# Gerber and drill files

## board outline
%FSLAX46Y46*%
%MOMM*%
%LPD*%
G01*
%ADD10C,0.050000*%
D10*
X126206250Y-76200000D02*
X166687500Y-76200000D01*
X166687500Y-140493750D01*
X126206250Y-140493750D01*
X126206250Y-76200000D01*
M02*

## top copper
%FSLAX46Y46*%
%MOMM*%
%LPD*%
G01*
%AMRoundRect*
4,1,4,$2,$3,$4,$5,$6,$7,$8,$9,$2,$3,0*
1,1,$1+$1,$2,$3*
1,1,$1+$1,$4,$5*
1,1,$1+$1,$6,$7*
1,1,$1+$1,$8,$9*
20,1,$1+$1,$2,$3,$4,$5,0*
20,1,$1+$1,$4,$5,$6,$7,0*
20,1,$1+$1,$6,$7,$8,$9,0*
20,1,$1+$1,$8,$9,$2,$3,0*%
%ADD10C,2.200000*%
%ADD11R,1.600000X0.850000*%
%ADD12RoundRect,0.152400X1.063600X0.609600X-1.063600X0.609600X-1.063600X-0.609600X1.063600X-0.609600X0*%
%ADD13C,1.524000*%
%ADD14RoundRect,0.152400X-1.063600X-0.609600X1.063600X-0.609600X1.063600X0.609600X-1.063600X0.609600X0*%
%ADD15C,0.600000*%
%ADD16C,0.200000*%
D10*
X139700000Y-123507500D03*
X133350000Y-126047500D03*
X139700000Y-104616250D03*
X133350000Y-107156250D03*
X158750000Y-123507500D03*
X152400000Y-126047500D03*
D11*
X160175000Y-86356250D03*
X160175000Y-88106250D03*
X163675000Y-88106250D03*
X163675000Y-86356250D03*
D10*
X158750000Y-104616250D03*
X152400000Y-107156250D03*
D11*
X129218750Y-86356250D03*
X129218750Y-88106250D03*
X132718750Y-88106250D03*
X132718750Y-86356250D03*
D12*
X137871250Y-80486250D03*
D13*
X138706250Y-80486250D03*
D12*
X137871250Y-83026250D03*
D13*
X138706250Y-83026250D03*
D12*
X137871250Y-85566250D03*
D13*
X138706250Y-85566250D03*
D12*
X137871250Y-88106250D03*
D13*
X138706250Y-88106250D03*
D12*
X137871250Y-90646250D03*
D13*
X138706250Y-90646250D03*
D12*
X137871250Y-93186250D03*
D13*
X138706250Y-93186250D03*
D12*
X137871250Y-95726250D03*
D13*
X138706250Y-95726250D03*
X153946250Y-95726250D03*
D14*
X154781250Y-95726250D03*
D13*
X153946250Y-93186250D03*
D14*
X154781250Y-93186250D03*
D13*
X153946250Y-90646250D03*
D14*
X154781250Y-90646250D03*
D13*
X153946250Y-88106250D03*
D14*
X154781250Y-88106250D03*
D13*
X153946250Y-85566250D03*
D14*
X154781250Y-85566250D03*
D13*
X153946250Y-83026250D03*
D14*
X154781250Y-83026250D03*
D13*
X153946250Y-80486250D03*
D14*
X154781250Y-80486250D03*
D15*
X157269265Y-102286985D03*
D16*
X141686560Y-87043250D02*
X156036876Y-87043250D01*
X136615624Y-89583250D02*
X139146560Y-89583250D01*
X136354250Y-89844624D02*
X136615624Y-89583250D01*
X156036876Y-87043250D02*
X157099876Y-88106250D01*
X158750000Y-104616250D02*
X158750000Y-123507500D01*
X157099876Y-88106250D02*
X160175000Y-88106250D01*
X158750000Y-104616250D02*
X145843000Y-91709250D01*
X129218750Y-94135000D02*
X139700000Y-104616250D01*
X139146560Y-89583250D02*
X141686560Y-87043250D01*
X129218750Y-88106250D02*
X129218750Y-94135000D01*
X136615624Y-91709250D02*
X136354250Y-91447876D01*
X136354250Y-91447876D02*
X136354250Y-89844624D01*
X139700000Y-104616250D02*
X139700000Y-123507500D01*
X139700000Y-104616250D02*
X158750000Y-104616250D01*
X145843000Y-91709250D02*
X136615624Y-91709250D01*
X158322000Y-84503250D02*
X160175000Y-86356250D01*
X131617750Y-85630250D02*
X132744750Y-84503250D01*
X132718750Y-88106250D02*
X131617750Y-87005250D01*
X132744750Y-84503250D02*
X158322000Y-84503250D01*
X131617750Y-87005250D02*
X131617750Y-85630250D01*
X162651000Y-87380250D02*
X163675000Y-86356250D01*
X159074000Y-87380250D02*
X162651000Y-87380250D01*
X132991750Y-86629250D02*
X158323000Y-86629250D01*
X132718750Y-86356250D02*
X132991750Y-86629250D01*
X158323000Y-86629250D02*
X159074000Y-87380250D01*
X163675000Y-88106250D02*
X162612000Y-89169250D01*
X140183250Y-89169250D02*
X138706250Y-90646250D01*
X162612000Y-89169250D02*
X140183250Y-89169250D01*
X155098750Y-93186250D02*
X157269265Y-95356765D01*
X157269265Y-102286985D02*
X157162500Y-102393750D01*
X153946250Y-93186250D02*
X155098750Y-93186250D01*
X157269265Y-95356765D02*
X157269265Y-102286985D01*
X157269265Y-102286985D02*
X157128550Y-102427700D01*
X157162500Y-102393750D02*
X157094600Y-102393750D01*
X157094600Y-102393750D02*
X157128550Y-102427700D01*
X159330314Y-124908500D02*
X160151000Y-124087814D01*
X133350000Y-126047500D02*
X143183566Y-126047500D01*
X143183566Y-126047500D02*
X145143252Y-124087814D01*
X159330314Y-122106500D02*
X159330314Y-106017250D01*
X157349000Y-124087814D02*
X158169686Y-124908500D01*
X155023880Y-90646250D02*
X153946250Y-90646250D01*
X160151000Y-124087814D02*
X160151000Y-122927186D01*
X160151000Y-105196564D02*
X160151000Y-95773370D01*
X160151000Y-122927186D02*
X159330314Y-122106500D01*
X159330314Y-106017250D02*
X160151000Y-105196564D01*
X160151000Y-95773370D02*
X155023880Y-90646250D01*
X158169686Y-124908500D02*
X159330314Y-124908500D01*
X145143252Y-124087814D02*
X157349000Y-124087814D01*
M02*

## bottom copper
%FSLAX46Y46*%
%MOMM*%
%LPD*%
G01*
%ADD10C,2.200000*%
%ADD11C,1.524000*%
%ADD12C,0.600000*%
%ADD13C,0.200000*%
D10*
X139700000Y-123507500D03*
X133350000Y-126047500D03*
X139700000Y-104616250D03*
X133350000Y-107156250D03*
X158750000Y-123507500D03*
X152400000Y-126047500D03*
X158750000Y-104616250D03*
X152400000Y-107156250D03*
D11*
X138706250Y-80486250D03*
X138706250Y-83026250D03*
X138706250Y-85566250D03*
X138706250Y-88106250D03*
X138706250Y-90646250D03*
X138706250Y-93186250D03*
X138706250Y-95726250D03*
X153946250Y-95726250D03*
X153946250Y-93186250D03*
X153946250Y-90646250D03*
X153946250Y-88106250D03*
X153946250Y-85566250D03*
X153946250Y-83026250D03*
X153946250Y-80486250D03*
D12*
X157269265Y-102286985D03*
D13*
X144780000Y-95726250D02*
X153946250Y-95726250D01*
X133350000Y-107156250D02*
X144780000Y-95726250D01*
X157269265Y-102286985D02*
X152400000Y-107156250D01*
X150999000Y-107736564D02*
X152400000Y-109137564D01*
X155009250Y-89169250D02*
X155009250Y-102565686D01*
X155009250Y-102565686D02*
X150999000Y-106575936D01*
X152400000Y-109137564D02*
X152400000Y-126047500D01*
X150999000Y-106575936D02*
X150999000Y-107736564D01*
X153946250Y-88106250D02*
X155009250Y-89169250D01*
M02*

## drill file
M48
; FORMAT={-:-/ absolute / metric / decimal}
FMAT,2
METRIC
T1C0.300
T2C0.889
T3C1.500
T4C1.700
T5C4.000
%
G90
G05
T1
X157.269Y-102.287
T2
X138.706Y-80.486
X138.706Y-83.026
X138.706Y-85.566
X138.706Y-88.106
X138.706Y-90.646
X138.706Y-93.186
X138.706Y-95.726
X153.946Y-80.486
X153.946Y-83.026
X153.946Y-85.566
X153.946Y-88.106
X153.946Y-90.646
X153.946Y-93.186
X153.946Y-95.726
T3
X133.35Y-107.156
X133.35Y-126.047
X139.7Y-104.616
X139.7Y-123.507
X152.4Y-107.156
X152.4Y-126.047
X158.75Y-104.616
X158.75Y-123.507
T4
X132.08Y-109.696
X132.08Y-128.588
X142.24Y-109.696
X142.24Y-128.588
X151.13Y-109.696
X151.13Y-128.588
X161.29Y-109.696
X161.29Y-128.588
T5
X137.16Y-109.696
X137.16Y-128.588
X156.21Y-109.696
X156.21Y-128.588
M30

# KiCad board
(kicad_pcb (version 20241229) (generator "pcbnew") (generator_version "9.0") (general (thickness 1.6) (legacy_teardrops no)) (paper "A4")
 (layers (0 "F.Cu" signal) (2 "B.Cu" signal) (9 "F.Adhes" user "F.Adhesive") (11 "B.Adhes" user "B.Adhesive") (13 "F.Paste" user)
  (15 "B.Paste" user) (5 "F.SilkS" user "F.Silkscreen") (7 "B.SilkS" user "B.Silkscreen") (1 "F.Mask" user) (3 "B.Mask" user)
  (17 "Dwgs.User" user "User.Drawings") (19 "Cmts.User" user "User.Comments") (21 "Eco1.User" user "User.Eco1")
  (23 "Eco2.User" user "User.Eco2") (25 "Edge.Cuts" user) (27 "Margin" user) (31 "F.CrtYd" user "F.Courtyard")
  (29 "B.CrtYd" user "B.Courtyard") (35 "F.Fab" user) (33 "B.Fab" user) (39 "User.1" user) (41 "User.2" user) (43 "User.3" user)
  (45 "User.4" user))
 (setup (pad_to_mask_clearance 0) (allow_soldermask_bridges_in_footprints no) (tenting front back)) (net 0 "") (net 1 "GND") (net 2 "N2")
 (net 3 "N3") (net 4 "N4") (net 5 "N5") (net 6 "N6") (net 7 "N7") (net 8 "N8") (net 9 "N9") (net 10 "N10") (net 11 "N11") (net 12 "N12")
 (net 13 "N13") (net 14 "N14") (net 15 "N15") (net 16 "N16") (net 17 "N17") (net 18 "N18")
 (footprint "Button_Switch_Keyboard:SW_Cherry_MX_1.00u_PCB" (layer "F.Cu") (at 139.7 123.5075)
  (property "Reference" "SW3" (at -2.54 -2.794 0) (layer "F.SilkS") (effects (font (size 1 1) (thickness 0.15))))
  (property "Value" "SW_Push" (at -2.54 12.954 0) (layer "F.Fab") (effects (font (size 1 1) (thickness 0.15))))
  (pad "" np_thru_hole circle (at -7.62 5.08) (size 1.7 1.7) (drill 1.7) (layers "*.Cu" "*.Mask"))
  (pad "" np_thru_hole circle (at -2.54 5.08) (size 4 4) (drill 4) (layers "*.Cu" "*.Mask"))
  (pad "" np_thru_hole circle (at 2.54 5.08) (size 1.7 1.7) (drill 1.7) (layers "*.Cu" "*.Mask"))
  (pad "1" thru_hole circle (at 0 0) (size 2.2 2.2) (drill 1.5) (layers "*.Cu" "*.Mask") (remove_unused_layers no) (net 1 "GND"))
  (pad "2" thru_hole circle (at -6.35 2.54) (size 2.2 2.2) (drill 1.5) (layers "*.Cu" "*.Mask") (remove_unused_layers no) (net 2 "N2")))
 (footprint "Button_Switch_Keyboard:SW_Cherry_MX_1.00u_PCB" (layer "F.Cu") (at 139.7 104.61625)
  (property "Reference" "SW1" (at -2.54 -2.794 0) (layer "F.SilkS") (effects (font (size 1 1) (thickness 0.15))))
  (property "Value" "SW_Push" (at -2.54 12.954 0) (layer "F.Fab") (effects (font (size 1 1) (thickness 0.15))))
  (pad "" np_thru_hole circle (at -7.62 5.08) (size 1.7 1.7) (drill 1.7) (layers "*.Cu" "*.Mask"))
  (pad "" np_thru_hole circle (at -2.54 5.08) (size 4 4) (drill 4) (layers "*.Cu" "*.Mask"))
  (pad "" np_thru_hole circle (at 2.54 5.08) (size 1.7 1.7) (drill 1.7) (layers "*.Cu" "*.Mask"))
  (pad "1" thru_hole circle (at 0 0) (size 2.2 2.2) (drill 1.5) (layers "*.Cu" "*.Mask") (remove_unused_layers no) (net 1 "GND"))
  (pad "2" thru_hole circle (at -6.35 2.54) (size 2.2 2.2) (drill 1.5) (layers "*.Cu" "*.Mask") (remove_unused_layers no) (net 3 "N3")))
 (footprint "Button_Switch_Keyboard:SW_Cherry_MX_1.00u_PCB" (layer "F.Cu") (at 158.75 123.5075)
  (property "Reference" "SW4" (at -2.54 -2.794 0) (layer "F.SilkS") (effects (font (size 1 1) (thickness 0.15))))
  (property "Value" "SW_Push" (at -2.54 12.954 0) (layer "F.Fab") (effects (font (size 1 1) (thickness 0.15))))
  (pad "" np_thru_hole circle (at -7.62 5.08) (size 1.7 1.7) (drill 1.7) (layers "*.Cu" "*.Mask"))
  (pad "" np_thru_hole circle (at -2.54 5.08) (size 4 4) (drill 4) (layers "*.Cu" "*.Mask"))
  (pad "" np_thru_hole circle (at 2.54 5.08) (size 1.7 1.7) (drill 1.7) (layers "*.Cu" "*.Mask"))
  (pad "1" thru_hole circle (at 0 0) (size 2.2 2.2) (drill 1.5) (layers "*.Cu" "*.Mask") (remove_unused_layers no) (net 1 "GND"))
  (pad "2" thru_hole circle (at -6.35 2.54) (size 2.2 2.2) (drill 1.5) (layers "*.Cu" "*.Mask") (remove_unused_layers no) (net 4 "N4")))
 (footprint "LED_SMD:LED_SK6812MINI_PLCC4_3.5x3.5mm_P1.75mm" (layer "F.Cu") (at 161.925 87.23125)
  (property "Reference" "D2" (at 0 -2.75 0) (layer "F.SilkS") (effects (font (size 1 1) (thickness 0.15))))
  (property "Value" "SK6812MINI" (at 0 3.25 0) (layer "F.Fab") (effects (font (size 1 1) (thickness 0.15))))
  (pad "1" smd rect (at -1.75 -0.875) (size 1.6 0.85) (layers "F.Cu" "F.Mask" "F.Paste") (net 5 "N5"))
  (pad "2" smd rect (at -1.75 0.875) (size 1.6 0.85) (layers "F.Cu" "F.Mask" "F.Paste") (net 1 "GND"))
  (pad "3" smd rect (at 1.75 0.875) (size 1.6 0.85) (layers "F.Cu" "F.Mask" "F.Paste") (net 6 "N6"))
  (pad "4" smd rect (at 1.75 -0.875) (size 1.6 0.85) (layers "F.Cu" "F.Mask" "F.Paste") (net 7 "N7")))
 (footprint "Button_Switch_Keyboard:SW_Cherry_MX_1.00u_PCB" (layer "F.Cu") (at 158.75 104.61625)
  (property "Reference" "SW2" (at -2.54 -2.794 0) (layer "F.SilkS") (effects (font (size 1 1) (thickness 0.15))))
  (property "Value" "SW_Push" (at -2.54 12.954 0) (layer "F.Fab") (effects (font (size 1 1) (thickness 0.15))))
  (pad "" np_thru_hole circle (at -7.62 5.08) (size 1.7 1.7) (drill 1.7) (layers "*.Cu" "*.Mask"))
  (pad "" np_thru_hole circle (at -2.54 5.08) (size 4 4) (drill 4) (layers "*.Cu" "*.Mask"))
  (pad "" np_thru_hole circle (at 2.54 5.08) (size 1.7 1.7) (drill 1.7) (layers "*.Cu" "*.Mask"))
  (pad "1" thru_hole circle (at 0 0) (size 2.2 2.2) (drill 1.5) (layers "*.Cu" "*.Mask") (remove_unused_layers no) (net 1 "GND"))
  (pad "2" thru_hole circle (at -6.35 2.54) (size 2.2 2.2) (drill 1.5) (layers "*.Cu" "*.Mask") (remove_unused_layers no) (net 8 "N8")))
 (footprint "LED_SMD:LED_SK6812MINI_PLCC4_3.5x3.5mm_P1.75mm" (layer "F.Cu") (at 130.96875 87.23125)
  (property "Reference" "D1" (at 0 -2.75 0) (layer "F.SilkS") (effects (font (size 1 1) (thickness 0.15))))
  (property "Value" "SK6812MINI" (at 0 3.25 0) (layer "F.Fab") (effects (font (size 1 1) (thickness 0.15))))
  (pad "1" smd rect (at -1.75 -0.875) (size 1.6 0.85) (layers "F.Cu" "F.Mask" "F.Paste") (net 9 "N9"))
  (pad "2" smd rect (at -1.75 0.875) (size 1.6 0.85) (layers "F.Cu" "F.Mask" "F.Paste") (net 1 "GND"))
  (pad "3" smd rect (at 1.75 0.875) (size 1.6 0.85) (layers "F.Cu" "F.Mask" "F.Paste") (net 5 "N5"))
  (pad "4" smd rect (at 1.75 -0.875) (size 1.6 0.85) (layers "F.Cu" "F.Mask" "F.Paste") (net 7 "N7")))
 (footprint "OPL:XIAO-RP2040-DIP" (layer "F.Cu") (at 146.32625 88.10625)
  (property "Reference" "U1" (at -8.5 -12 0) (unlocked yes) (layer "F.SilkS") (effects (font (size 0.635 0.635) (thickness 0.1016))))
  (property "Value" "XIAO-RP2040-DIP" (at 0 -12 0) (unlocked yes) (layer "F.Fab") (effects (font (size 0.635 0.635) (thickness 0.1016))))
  (pad "1" smd roundrect (at -8.455 -7.62 180) (size 2.432 1.524) (layers "F.Cu" "F.Mask") (roundrect_rratio 0.1) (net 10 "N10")
   (thermal_bridge_angle 45))
  (pad "1" thru_hole circle (at -7.62 -7.62 180) (size 1.524 1.524) (drill 0.889) (layers "*.Cu" "*.Mask") (remove_unused_layers no)
   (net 10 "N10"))
  (pad "2" smd roundrect (at -8.455 -5.08 180) (size 2.432 1.524) (layers "F.Cu" "F.Mask") (roundrect_rratio 0.1) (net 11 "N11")
   (thermal_bridge_angle 45))
  (pad "2" thru_hole circle (at -7.62 -5.08 180) (size 1.524 1.524) (drill 0.889) (layers "*.Cu" "*.Mask") (remove_unused_layers no)
   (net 11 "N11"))
  (pad "3" smd roundrect (at -8.455 -2.54 180) (size 2.432 1.524) (layers "F.Cu" "F.Mask") (roundrect_rratio 0.1) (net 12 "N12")
   (thermal_bridge_angle 45))
  (pad "3" thru_hole circle (at -7.62 -2.54 180) (size 1.524 1.524) (drill 0.889) (layers "*.Cu" "*.Mask") (remove_unused_layers no)
   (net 12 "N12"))
  (pad "4" smd roundrect (at -8.455 0 180) (size 2.432 1.524) (layers "F.Cu" "F.Mask") (roundrect_rratio 0.1) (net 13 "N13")
   (thermal_bridge_angle 45))
  (pad "4" thru_hole circle (at -7.62 0 180) (size 1.524 1.524) (drill 0.889) (layers "*.Cu" "*.Mask") (remove_unused_layers no)
   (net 13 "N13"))
  (pad "5" smd roundrect (at -8.455 2.54 180) (size 2.432 1.524) (layers "F.Cu" "F.Mask") (roundrect_rratio 0.1) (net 6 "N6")
   (thermal_bridge_angle 45))
  (pad "5" thru_hole circle (at -7.62 2.54 180) (size 1.524 1.524) (drill 0.889) (layers "*.Cu" "*.Mask") (remove_unused_layers no)
   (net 6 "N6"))
  (pad "6" smd roundrect (at -8.455 5.08 180) (size 2.432 1.524) (layers "F.Cu" "F.Mask") (roundrect_rratio 0.1) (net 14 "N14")
   (thermal_bridge_angle 45))
  (pad "6" thru_hole circle (at -7.62 5.08 180) (size 1.524 1.524) (drill 0.889) (layers "*.Cu" "*.Mask") (remove_unused_layers no)
   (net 14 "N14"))
  (pad "7" smd roundrect (at -8.455 7.62 180) (size 2.432 1.524) (layers "F.Cu" "F.Mask") (roundrect_rratio 0.1) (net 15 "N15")
   (thermal_bridge_angle 45))
  (pad "7" thru_hole circle (at -7.62 7.62 180) (size 1.524 1.524) (drill 0.889) (layers "*.Cu" "*.Mask") (remove_unused_layers no)
   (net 15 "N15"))
  (pad "8" thru_hole circle (at 7.62 7.62) (size 1.524 1.524) (drill 0.889) (layers "*.Cu" "*.Mask") (remove_unused_layers no) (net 3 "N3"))
  (pad "8" smd roundrect (at 8.455 7.62) (size 2.432 1.524) (layers "F.Cu" "F.Mask") (roundrect_rratio 0.1) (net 3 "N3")
   (thermal_bridge_angle 45))
  (pad "9" thru_hole circle (at 7.62 5.08) (size 1.524 1.524) (drill 0.889) (layers "*.Cu" "*.Mask") (remove_unused_layers no) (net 8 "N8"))
  (pad "9" smd roundrect (at 8.455 5.08) (size 2.432 1.524) (layers "F.Cu" "F.Mask") (roundrect_rratio 0.1) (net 8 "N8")
   (thermal_bridge_angle 45))
  (pad "10" thru_hole circle (at 7.62 2.54) (size 1.524 1.524) (drill 0.889) (layers "*.Cu" "*.Mask") (remove_unused_layers no) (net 2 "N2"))
  (pad "10" smd roundrect (at 8.455 2.54) (size 2.432 1.524) (layers "F.Cu" "F.Mask") (roundrect_rratio 0.1) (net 2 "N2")
   (thermal_bridge_angle 45))
  (pad "11" thru_hole circle (at 7.62 0) (size 1.524 1.524) (drill 0.889) (layers "*.Cu" "*.Mask") (remove_unused_layers no) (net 4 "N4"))
  (pad "11" smd roundrect (at 8.455 0) (size 2.432 1.524) (layers "F.Cu" "F.Mask") (roundrect_rratio 0.1) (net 4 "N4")
   (thermal_bridge_angle 45))
  (pad "12" thru_hole circle (at 7.62 -2.54) (size 1.524 1.524) (drill 0.889) (layers "*.Cu" "*.Mask") (remove_unused_layers no)
   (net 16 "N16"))
  (pad "12" smd roundrect (at 8.455 -2.54) (size 2.432 1.524) (layers "F.Cu" "F.Mask") (roundrect_rratio 0.1) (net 16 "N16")
   (thermal_bridge_angle 45))
  (pad "13" thru_hole circle (at 7.62 -5.08) (size 1.524 1.524) (drill 0.889) (layers "*.Cu" "*.Mask") (remove_unused_layers no)
   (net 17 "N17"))
  (pad "13" smd roundrect (at 8.455 -5.08) (size 2.432 1.524) (layers "F.Cu" "F.Mask") (roundrect_rratio 0.1) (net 17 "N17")
   (thermal_bridge_angle 45))
  (pad "14" thru_hole circle (at 7.62 -7.62) (size 1.524 1.524) (drill 0.889) (layers "*.Cu" "*.Mask") (remove_unused_layers no)
   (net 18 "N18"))
  (pad "14" smd roundrect (at 8.455 -7.62) (size 2.432 1.524) (layers "F.Cu" "F.Mask") (roundrect_rratio 0.1) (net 18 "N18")
   (thermal_bridge_angle 45)))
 (gr_rect (start 126.20625 76.2) (end 166.6875 140.49375) (stroke (width 0.05) (type default)) (fill no) (layer "Edge.Cuts"))
 (segment (start 141.68656 87.04325) (end 156.036876 87.04325) (width 0.2) (layer "F.Cu") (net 1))
 (segment (start 136.615624 89.58325) (end 139.14656 89.58325) (width 0.2) (layer "F.Cu") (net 1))
 (segment (start 136.35425 89.844624) (end 136.615624 89.58325) (width 0.2) (layer "F.Cu") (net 1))
 (segment (start 156.036876 87.04325) (end 157.099876 88.10625) (width 0.2) (layer "F.Cu") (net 1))
 (segment (start 158.75 104.61625) (end 158.75 123.5075) (width 0.2) (layer "F.Cu") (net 1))
 (segment (start 157.099876 88.10625) (end 160.175 88.10625) (width 0.2) (layer "F.Cu") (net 1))
 (segment (start 158.75 104.61625) (end 145.843 91.70925) (width 0.2) (layer "F.Cu") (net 1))
 (segment (start 129.21875 94.135) (end 139.7 104.61625) (width 0.2) (layer "F.Cu") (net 1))
 (segment (start 139.14656 89.58325) (end 141.68656 87.04325) (width 0.2) (layer "F.Cu") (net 1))
 (segment (start 129.21875 88.10625) (end 129.21875 94.135) (width 0.2) (layer "F.Cu") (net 1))
 (segment (start 136.615624 91.70925) (end 136.35425 91.447876) (width 0.2) (layer "F.Cu") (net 1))
 (segment (start 136.35425 91.447876) (end 136.35425 89.844624) (width 0.2) (layer "F.Cu") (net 1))
 (segment (start 139.7 104.61625) (end 139.7 123.5075) (width 0.2) (layer "F.Cu") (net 1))
 (segment (start 139.7 104.61625) (end 158.75 104.61625) (width 0.2) (layer "F.Cu") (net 1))
 (segment (start 145.843 91.70925) (end 136.615624 91.70925) (width 0.2) (layer "F.Cu") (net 1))
 (segment (start 158.322 84.50325) (end 160.175 86.35625) (width 0.2) (layer "F.Cu") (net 5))
 (segment (start 131.61775 85.63025) (end 132.74475 84.50325) (width 0.2) (layer "F.Cu") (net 5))
 (segment (start 132.71875 88.10625) (end 131.61775 87.00525) (width 0.2) (layer "F.Cu") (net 5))
 (segment (start 132.74475 84.50325) (end 158.322 84.50325) (width 0.2) (layer "F.Cu") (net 5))
 (segment (start 131.61775 87.00525) (end 131.61775 85.63025) (width 0.2) (layer "F.Cu") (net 5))
 (segment (start 162.651 87.38025) (end 163.675 86.35625) (width 0.2) (layer "F.Cu") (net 7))
 (segment (start 159.074 87.38025) (end 162.651 87.38025) (width 0.2) (layer "F.Cu") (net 7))
 (segment (start 132.99175 86.62925) (end 158.323 86.62925) (width 0.2) (layer "F.Cu") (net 7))
 (segment (start 132.71875 86.35625) (end 132.99175 86.62925) (width 0.2) (layer "F.Cu") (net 7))
 (segment (start 158.323 86.62925) (end 159.074 87.38025) (width 0.2) (layer "F.Cu") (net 7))
 (segment (start 163.675 88.10625) (end 162.612 89.16925) (width 0.2) (layer "F.Cu") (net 6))
 (segment (start 140.18325 89.16925) (end 138.70625 90.64625) (width 0.2) (layer "F.Cu") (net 6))
 (segment (start 162.612 89.16925) (end 140.18325 89.16925) (width 0.2) (layer "F.Cu") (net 6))
 (segment (start 144.78 95.72625) (end 153.94625 95.72625) (width 0.2) (layer "B.Cu") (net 3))
 (segment (start 133.35 107.15625) (end 144.78 95.72625) (width 0.2) (layer "B.Cu") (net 3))
 (segment (start 155.09875 93.18625) (end 157.269265 95.356765) (width 0.2) (layer "F.Cu") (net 8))
 (segment (start 157.269265 102.286985) (end 157.1625 102.39375) (width 0.2) (layer "F.Cu") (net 8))
 (segment (start 153.94625 93.18625) (end 155.09875 93.18625) (width 0.2) (layer "F.Cu") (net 8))
 (segment (start 157.269265 95.356765) (end 157.269265 102.286985) (width 0.2) (layer "F.Cu") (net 8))
 (segment (start 157.269265 102.286985) (end 157.12855 102.4277) (width 0.2) (layer "F.Cu") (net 8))
 (segment (start 157.1625 102.39375) (end 157.0946 102.39375) (width 0.2) (layer "F.Cu") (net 8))
 (segment (start 157.0946 102.39375) (end 157.12855 102.4277) (width 0.2) (layer "F.Cu") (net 8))
 (via (at 157.269265 102.286985) (size 0.6) (drill 0.3) (layers "F.Cu" "B.Cu") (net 8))
 (segment (start 157.269265 102.286985) (end 152.4 107.15625) (width 0.2) (layer "B.Cu") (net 8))
 (segment (start 159.330314 124.9085) (end 160.151 124.087814) (width 0.2) (layer "F.Cu") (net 2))
 (segment (start 133.35 126.0475) (end 143.183566 126.0475) (width 0.2) (layer "F.Cu") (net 2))
 (segment (start 143.183566 126.0475) (end 145.143252 124.087814) (width 0.2) (layer "F.Cu") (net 2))
 (segment (start 159.330314 122.1065) (end 159.330314 106.01725) (width 0.2) (layer "F.Cu") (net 2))
 (segment (start 157.349 124.087814) (end 158.169686 124.9085) (width 0.2) (layer "F.Cu") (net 2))
 (segment (start 155.02388 90.64625) (end 153.94625 90.64625) (width 0.2) (layer "F.Cu") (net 2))
 (segment (start 160.151 124.087814) (end 160.151 122.927186) (width 0.2) (layer "F.Cu") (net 2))
 (segment (start 160.151 105.196564) (end 160.151 95.77337) (width 0.2) (layer "F.Cu") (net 2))
 (segment (start 160.151 122.927186) (end 159.330314 122.1065) (width 0.2) (layer "F.Cu") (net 2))
 (segment (start 159.330314 106.01725) (end 160.151 105.196564) (width 0.2) (layer "F.Cu") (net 2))
 (segment (start 160.151 95.77337) (end 155.02388 90.64625) (width 0.2) (layer "F.Cu") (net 2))
 (segment (start 158.169686 124.9085) (end 159.330314 124.9085) (width 0.2) (layer "F.Cu") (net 2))
 (segment (start 145.143252 124.087814) (end 157.349 124.087814) (width 0.2) (layer "F.Cu") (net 2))
 (segment (start 150.999 107.736564) (end 152.4 109.137564) (width 0.2) (layer "B.Cu") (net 4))
 (segment (start 155.00925 89.16925) (end 155.00925 102.565686) (width 0.2) (layer "B.Cu") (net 4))
 (segment (start 155.00925 102.565686) (end 150.999 106.575936) (width 0.2) (layer "B.Cu") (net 4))
 (segment (start 152.4 109.137564) (end 152.4 126.0475) (width 0.2) (layer "B.Cu") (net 4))
 (segment (start 150.999 106.575936) (end 150.999 107.736564) (width 0.2) (layer "B.Cu") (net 4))
 (segment (start 153.94625 88.10625) (end 155.00925 89.16925) (width 0.2) (layer "B.Cu") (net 4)))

